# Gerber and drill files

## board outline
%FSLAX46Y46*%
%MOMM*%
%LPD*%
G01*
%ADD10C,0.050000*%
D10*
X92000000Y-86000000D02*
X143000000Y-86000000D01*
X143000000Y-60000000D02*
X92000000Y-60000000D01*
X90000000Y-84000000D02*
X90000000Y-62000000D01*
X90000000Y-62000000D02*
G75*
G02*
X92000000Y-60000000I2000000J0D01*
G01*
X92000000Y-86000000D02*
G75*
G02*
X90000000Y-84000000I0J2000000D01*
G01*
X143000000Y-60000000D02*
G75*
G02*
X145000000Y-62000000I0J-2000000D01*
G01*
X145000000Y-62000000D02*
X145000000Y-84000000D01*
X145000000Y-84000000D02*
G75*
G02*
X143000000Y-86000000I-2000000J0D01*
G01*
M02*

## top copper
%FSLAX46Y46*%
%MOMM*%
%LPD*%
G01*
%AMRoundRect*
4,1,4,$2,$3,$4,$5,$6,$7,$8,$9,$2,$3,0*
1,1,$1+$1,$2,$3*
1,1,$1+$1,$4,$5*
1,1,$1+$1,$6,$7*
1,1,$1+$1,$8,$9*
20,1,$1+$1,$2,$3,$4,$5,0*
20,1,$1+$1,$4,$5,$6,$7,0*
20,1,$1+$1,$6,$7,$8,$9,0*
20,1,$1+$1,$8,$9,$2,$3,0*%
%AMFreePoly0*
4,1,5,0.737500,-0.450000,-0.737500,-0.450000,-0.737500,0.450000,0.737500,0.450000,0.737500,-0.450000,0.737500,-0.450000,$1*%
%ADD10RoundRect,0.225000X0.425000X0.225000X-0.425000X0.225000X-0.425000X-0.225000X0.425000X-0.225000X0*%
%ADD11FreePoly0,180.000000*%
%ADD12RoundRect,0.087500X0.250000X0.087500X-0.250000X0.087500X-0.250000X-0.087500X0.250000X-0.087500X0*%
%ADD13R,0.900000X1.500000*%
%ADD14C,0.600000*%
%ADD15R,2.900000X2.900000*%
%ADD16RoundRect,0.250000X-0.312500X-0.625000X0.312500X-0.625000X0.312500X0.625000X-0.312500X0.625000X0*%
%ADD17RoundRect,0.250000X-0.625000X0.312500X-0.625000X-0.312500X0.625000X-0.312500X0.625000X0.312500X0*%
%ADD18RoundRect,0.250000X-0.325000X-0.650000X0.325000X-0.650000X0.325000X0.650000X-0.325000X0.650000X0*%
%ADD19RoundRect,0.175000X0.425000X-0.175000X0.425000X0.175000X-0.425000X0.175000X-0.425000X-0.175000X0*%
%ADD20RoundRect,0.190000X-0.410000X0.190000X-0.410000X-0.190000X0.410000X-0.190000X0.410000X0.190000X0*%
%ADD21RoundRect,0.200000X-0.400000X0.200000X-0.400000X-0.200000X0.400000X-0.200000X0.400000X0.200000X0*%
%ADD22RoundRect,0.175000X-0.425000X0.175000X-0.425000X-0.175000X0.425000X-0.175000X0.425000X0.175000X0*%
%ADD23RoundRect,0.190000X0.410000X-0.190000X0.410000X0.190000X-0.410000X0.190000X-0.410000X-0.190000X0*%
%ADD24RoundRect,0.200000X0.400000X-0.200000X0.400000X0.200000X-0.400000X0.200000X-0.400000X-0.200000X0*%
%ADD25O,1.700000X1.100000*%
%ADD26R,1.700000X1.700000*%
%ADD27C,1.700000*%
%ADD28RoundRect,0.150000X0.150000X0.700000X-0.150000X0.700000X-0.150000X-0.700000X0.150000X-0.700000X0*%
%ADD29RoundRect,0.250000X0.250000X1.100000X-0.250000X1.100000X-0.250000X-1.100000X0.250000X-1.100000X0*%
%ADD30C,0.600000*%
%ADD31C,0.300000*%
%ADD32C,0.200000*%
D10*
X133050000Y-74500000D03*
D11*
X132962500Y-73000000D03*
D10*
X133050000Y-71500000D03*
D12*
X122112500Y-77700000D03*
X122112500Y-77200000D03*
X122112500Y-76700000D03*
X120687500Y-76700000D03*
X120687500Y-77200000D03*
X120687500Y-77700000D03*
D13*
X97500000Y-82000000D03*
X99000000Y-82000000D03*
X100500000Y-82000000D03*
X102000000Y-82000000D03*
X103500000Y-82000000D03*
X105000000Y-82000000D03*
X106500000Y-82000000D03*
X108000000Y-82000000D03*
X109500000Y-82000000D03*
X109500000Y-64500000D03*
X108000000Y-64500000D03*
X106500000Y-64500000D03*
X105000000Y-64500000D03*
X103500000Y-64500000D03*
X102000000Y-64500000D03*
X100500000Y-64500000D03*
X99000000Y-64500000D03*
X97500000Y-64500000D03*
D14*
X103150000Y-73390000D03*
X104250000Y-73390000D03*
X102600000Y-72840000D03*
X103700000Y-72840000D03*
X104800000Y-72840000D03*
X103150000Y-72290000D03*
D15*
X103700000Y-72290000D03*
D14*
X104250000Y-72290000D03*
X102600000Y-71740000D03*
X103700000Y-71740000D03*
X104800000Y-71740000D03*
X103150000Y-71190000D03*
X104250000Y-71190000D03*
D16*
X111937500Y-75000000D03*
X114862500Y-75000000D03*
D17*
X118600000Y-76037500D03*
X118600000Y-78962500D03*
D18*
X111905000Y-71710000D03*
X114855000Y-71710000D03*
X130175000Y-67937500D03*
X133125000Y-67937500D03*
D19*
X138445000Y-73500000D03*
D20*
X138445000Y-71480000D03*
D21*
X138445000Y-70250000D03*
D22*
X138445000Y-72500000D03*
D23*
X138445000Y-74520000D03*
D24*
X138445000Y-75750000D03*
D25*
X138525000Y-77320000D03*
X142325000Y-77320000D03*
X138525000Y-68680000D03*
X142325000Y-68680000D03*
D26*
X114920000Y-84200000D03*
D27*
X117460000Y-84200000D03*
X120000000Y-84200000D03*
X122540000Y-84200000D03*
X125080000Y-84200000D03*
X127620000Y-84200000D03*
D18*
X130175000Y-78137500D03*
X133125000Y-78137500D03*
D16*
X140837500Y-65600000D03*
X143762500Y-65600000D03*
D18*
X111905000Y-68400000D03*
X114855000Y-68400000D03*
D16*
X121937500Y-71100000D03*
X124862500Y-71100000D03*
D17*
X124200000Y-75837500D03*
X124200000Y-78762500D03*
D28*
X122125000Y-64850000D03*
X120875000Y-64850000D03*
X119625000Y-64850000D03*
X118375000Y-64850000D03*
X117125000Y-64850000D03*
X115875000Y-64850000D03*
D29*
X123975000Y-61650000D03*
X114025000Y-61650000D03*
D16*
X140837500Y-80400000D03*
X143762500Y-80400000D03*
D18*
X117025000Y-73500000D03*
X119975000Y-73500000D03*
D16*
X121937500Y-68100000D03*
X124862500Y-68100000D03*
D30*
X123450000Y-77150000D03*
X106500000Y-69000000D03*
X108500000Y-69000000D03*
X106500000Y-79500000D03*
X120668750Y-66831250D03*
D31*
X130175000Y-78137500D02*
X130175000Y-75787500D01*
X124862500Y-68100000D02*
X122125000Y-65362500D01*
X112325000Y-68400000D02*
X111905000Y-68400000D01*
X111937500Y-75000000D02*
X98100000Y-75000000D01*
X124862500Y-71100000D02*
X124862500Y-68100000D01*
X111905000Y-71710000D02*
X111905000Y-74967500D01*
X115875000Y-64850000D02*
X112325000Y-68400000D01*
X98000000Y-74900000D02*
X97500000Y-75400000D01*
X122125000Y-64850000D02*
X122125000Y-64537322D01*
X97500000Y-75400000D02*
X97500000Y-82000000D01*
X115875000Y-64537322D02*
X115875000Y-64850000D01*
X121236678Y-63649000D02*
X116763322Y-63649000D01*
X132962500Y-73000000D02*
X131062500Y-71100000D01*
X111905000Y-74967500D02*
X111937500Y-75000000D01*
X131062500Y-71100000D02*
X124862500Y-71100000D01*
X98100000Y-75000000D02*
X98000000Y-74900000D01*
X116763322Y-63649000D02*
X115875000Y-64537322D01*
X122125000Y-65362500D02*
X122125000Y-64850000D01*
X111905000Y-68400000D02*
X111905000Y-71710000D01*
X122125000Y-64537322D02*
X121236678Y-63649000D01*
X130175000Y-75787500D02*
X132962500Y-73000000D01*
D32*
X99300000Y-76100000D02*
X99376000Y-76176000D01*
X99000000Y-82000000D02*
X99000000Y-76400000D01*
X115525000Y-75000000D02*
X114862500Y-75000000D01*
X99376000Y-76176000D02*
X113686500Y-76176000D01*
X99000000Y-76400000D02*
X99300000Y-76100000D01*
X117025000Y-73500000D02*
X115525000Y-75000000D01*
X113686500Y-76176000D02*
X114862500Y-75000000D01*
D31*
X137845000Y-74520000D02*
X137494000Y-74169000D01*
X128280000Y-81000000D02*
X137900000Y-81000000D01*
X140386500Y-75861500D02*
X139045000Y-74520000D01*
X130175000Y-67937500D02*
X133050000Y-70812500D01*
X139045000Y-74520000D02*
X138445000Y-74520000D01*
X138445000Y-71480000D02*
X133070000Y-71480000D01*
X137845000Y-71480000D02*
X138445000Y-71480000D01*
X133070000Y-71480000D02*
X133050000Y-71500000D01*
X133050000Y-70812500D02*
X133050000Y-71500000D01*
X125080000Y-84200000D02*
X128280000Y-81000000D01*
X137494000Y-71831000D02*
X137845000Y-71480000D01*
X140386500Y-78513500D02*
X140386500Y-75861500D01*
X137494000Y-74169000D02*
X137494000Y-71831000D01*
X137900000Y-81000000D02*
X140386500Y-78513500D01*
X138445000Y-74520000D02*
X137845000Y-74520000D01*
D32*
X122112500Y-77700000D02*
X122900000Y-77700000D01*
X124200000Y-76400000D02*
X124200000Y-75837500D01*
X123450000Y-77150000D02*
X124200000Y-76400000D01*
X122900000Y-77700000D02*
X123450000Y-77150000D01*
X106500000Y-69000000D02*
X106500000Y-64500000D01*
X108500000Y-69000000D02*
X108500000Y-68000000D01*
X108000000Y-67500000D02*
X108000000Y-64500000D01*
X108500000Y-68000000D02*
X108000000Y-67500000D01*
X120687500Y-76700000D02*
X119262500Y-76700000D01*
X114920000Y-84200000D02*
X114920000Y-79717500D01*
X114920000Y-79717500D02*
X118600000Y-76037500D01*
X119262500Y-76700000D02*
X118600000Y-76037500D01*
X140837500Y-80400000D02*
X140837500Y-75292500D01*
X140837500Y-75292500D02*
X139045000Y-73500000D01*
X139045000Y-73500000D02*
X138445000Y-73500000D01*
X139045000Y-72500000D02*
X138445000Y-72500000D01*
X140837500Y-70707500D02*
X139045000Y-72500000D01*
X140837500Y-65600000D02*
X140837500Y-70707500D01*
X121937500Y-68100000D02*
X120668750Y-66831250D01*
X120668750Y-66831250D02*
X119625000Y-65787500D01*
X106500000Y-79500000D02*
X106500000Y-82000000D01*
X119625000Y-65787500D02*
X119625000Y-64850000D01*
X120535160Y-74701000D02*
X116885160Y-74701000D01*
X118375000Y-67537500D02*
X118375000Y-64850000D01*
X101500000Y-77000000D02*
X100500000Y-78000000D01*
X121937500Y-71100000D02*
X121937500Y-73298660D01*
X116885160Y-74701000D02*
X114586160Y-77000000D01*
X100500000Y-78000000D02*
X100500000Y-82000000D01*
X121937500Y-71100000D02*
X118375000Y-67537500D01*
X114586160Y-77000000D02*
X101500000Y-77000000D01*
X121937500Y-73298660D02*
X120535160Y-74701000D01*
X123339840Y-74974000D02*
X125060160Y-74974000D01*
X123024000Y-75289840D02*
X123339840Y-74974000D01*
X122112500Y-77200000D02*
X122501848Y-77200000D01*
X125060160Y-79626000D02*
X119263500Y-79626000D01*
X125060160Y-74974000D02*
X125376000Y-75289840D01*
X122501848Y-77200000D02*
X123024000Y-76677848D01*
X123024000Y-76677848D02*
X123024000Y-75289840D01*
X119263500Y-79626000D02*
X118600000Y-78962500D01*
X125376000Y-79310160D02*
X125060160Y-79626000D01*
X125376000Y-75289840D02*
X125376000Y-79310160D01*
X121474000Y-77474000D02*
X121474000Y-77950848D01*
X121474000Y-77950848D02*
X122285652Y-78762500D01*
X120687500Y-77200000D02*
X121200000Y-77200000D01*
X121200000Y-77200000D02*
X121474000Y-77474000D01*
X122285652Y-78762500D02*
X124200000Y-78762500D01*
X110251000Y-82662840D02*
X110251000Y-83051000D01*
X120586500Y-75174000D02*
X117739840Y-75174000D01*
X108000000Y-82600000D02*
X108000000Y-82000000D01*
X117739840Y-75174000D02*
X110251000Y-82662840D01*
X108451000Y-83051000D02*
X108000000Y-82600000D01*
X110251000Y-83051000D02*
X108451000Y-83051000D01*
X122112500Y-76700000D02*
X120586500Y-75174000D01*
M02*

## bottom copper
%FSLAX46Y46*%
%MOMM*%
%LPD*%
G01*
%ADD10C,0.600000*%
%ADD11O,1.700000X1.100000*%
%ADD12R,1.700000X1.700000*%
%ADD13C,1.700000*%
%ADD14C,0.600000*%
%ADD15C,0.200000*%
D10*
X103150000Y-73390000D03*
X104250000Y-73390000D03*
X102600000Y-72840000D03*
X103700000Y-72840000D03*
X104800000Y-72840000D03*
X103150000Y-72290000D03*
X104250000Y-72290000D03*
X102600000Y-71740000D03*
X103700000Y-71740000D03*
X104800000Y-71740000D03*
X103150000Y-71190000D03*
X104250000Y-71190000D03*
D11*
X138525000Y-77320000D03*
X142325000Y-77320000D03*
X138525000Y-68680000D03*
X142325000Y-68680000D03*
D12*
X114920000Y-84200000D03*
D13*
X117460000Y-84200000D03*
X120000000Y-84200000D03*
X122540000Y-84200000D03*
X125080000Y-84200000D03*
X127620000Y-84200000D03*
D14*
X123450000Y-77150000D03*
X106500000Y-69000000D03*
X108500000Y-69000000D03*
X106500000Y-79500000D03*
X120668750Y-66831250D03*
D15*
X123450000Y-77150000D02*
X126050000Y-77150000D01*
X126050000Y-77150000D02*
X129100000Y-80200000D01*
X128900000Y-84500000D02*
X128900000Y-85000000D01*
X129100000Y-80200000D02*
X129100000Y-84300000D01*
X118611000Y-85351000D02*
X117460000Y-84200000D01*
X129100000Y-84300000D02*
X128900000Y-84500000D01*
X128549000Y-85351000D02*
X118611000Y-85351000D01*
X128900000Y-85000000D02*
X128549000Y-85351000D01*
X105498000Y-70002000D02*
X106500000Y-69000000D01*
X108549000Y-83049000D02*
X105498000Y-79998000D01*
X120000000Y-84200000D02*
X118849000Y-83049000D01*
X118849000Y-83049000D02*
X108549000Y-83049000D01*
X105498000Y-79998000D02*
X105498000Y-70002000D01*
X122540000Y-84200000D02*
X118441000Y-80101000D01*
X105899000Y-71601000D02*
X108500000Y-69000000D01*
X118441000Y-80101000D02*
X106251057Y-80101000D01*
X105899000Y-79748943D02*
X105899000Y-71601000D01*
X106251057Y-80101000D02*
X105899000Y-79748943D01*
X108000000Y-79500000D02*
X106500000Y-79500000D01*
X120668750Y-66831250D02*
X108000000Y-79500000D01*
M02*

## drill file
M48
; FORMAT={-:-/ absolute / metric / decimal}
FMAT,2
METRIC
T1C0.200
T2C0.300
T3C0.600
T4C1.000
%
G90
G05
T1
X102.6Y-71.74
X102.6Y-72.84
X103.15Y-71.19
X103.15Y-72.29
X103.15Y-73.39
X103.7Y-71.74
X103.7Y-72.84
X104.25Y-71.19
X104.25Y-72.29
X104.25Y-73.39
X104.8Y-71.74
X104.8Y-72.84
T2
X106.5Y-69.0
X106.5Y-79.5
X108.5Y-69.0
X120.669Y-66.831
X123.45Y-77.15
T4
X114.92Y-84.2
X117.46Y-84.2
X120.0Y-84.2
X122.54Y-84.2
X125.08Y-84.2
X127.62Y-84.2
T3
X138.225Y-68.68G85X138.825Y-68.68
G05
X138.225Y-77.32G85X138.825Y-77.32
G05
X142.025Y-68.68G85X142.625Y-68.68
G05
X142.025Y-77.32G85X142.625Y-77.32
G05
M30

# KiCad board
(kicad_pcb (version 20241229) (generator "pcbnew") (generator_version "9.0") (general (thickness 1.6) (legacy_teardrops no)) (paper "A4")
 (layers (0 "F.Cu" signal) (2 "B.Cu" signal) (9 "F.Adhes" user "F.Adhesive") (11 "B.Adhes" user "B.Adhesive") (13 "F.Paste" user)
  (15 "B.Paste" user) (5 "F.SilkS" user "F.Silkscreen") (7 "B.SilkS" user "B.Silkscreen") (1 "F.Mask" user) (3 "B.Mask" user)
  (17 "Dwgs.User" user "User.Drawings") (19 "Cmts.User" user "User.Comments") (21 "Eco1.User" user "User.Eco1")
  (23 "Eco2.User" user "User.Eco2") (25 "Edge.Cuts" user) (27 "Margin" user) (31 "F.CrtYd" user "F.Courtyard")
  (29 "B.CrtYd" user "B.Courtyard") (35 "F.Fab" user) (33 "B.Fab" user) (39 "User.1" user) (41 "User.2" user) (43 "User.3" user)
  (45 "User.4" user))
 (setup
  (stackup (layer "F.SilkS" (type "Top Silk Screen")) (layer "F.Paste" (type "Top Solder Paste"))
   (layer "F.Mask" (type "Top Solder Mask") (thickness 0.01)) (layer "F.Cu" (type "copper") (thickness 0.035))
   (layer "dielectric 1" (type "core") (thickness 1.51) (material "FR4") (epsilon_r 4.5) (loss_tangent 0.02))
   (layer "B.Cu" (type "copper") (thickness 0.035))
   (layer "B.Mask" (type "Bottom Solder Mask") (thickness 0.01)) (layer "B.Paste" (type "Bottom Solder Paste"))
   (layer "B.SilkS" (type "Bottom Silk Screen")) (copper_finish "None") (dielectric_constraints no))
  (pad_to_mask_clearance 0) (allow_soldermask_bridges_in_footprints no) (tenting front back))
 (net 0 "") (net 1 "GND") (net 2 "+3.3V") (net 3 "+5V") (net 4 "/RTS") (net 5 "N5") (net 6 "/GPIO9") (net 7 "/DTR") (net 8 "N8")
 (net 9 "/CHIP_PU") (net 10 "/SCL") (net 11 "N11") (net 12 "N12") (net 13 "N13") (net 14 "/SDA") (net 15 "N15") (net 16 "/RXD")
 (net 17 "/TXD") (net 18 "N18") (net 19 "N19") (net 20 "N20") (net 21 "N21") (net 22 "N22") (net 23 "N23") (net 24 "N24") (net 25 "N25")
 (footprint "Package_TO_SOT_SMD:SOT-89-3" (layer "F.Cu") (at 131.1 73 180)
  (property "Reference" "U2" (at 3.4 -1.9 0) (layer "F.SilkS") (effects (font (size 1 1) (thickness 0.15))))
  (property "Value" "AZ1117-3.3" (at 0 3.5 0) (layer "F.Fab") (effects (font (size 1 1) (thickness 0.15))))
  (pad "1" smd roundrect (at -1.95 -1.5 180) (size 1.3 0.9) (layers "F.Cu" "F.Mask" "F.Paste") (roundrect_rratio 0.25) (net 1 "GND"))
  (pad "2" smd custom (at -1.8625 0 180) (size 1.475 0.9) (layers "F.Cu" "F.Mask" "F.Paste") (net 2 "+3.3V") (zone_connect 2)
   (thermal_bridge_angle 45) (options (clearance outline) (anchor rect)) (primitives))
  (pad "3" smd roundrect (at -1.95 1.5 180) (size 1.3 0.9) (layers "F.Cu" "F.Mask" "F.Paste") (roundrect_rratio 0.25) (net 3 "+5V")))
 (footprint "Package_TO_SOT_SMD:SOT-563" (layer "F.Cu") (at 121.4 77.2 180)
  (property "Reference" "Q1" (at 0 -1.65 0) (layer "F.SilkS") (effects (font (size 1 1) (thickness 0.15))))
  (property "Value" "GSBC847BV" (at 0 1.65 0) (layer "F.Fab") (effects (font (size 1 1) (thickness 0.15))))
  (pad "1" smd roundrect (at -0.7125 -0.5 180) (size 0.675 0.35) (layers "F.Cu" "F.Mask" "F.Paste") (roundrect_rratio 0.25) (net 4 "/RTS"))
  (pad "2" smd roundrect (at -0.7125 0 180) (size 0.675 0.35) (layers "F.Cu" "F.Mask" "F.Paste") (roundrect_rratio 0.25) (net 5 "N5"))
  (pad "3" smd roundrect (at -0.7125 0.5 180) (size 0.675 0.35) (layers "F.Cu" "F.Mask" "F.Paste") (roundrect_rratio 0.25) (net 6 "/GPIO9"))
  (pad "4" smd roundrect (at 0.7125 0.5 180) (size 0.675 0.35) (layers "F.Cu" "F.Mask" "F.Paste") (roundrect_rratio 0.25) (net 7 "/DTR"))
  (pad "5" smd roundrect (at 0.7125 0 180) (size 0.675 0.35) (layers "F.Cu" "F.Mask" "F.Paste") (roundrect_rratio 0.25) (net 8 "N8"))
  (pad "6" smd roundrect (at 0.7125 -0.5 180) (size 0.675 0.35) (layers "F.Cu" "F.Mask" "F.Paste") (roundrect_rratio 0.25)
   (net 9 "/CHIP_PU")))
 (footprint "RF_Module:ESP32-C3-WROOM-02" (layer "F.Cu") (at 103.5 73.25 90)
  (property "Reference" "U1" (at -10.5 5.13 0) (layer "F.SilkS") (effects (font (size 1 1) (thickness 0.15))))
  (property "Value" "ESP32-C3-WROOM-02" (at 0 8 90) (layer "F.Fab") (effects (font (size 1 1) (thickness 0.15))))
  (pad "" smd rect (at -0.14 -0.9 90) (size 0.7 0.7) (layers "F.Paste"))
  (pad "" smd rect (at -0.14 0.2 90) (size 0.7 0.7) (layers "F.Paste"))
  (pad "" smd rect (at -0.14 1.3 90) (size 0.7 0.7) (layers "F.Paste"))
  (pad "" smd rect (at 0.96 -0.9 90) (size 0.7 0.7) (layers "F.Paste"))
  (pad "" smd rect (at 0.96 0.2 90) (size 0.7 0.7) (layers "F.Paste"))
  (pad "" smd rect (at 0.96 1.3 90) (size 0.7 0.7) (layers "F.Paste"))
  (pad "" smd rect (at 2.06 -0.9 90) (size 0.7 0.7) (layers "F.Paste"))
  (pad "" smd rect (at 2.06 0.2 90) (size 0.7 0.7) (layers "F.Paste"))
  (pad "" smd rect (at 2.06 1.3 90) (size 0.7 0.7) (layers "F.Paste"))
  (pad "1" smd rect (at -8.75 -6 90) (size 1.5 0.9) (layers "F.Cu" "F.Mask" "F.Paste") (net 2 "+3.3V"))
  (pad "2" smd rect (at -8.75 -4.5 90) (size 1.5 0.9) (layers "F.Cu" "F.Mask" "F.Paste") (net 9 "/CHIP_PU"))
  (pad "3" smd rect (at -8.75 -3 90) (size 1.5 0.9) (layers "F.Cu" "F.Mask" "F.Paste") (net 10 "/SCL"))
  (pad "4" smd rect (at -8.75 -1.5 90) (size 1.5 0.9) (layers "F.Cu" "F.Mask" "F.Paste") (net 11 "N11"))
  (pad "5" smd rect (at -8.75 0 90) (size 1.5 0.9) (layers "F.Cu" "F.Mask" "F.Paste") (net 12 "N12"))
  (pad "6" smd rect (at -8.75 1.5 90) (size 1.5 0.9) (layers "F.Cu" "F.Mask" "F.Paste") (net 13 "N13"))
  (pad "7" smd rect (at -8.75 3 90) (size 1.5 0.9) (layers "F.Cu" "F.Mask" "F.Paste") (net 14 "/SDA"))
  (pad "8" smd rect (at -8.75 4.5 90) (size 1.5 0.9) (layers "F.Cu" "F.Mask" "F.Paste") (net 6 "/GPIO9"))
  (pad "9" smd rect (at -8.75 6 90) (size 1.5 0.9) (layers "F.Cu" "F.Mask" "F.Paste") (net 1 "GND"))
  (pad "10" smd rect (at 8.75 6 90) (size 1.5 0.9) (layers "F.Cu" "F.Mask" "F.Paste") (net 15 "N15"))
  (pad "11" smd rect (at 8.75 4.5 90) (size 1.5 0.9) (layers "F.Cu" "F.Mask" "F.Paste") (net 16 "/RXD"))
  (pad "12" smd rect (at 8.75 3 90) (size 1.5 0.9) (layers "F.Cu" "F.Mask" "F.Paste") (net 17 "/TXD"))
  (pad "13" smd rect (at 8.75 1.5 90) (size 1.5 0.9) (layers "F.Cu" "F.Mask" "F.Paste") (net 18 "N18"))
  (pad "14" smd rect (at 8.75 0 90) (size 1.5 0.9) (layers "F.Cu" "F.Mask" "F.Paste") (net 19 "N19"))
  (pad "15" smd rect (at 8.75 -1.5 90) (size 1.5 0.9) (layers "F.Cu" "F.Mask" "F.Paste") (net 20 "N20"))
  (pad "16" smd rect (at 8.75 -3 90) (size 1.5 0.9) (layers "F.Cu" "F.Mask" "F.Paste") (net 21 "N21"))
  (pad "17" smd rect (at 8.75 -4.5 90) (size 1.5 0.9) (layers "F.Cu" "F.Mask" "F.Paste") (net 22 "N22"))
  (pad "18" smd rect (at 8.75 -6 90) (size 1.5 0.9) (layers "F.Cu" "F.Mask" "F.Paste") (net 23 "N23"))
  (pad "19" thru_hole circle (at -0.14 -0.35 90) (size 0.6 0.6) (drill 0.2) (layers "*.Cu" "F.Mask") (remove_unused_layers no) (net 1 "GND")
   (zone_connect 2))
  (pad "19" thru_hole circle (at -0.14 0.75 90) (size 0.6 0.6) (drill 0.2) (layers "*.Cu" "F.Mask") (remove_unused_layers no) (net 1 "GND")
   (zone_connect 2))
  (pad "19" thru_hole circle (at 0.41 -0.9 90) (size 0.6 0.6) (drill 0.2) (layers "*.Cu" "F.Mask") (remove_unused_layers no) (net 1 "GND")
   (zone_connect 2))
  (pad "19" thru_hole circle (at 0.41 0.2 90) (size 0.6 0.6) (drill 0.2) (layers "*.Cu" "F.Mask") (remove_unused_layers no) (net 1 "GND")
   (zone_connect 2))
  (pad "19" thru_hole circle (at 0.41 1.3 90) (size 0.6 0.6) (drill 0.2) (layers "*.Cu" "F.Mask") (remove_unused_layers no) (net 1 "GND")
   (zone_connect 2))
  (pad "19" thru_hole circle (at 0.96 -0.35 90) (size 0.6 0.6) (drill 0.2) (layers "*.Cu" "F.Mask") (remove_unused_layers no) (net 1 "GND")
   (zone_connect 2))
  (pad "19" smd rect (at 0.96 0.2 90) (size 2.9 2.9) (layers "F.Cu" "F.Mask") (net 1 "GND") (zone_connect 2))
  (pad "19" thru_hole circle (at 0.96 0.75 90) (size 0.6 0.6) (drill 0.2) (layers "*.Cu" "F.Mask") (remove_unused_layers no) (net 1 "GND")
   (zone_connect 2))
  (pad "19" thru_hole circle (at 1.51 -0.9 90) (size 0.6 0.6) (drill 0.2) (layers "*.Cu" "F.Mask") (remove_unused_layers no) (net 1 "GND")
   (zone_connect 2))
  (pad "19" thru_hole circle (at 1.51 0.2 90) (size 0.6 0.6) (drill 0.2) (layers "*.Cu" "F.Mask") (remove_unused_layers no) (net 1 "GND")
   (zone_connect 2))
  (pad "19" thru_hole circle (at 1.51 1.3 90) (size 0.6 0.6) (drill 0.2) (layers "*.Cu" "F.Mask") (remove_unused_layers no) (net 1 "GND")
   (zone_connect 2))
  (pad "19" thru_hole circle (at 2.06 -0.35 90) (size 0.6 0.6) (drill 0.2) (layers "*.Cu" "F.Mask") (remove_unused_layers no) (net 1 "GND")
   (zone_connect 2))
  (pad "19" thru_hole circle (at 2.06 0.75 90) (size 0.6 0.6) (drill 0.2) (layers "*.Cu" "F.Mask") (remove_unused_layers no) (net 1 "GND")
   (zone_connect 2))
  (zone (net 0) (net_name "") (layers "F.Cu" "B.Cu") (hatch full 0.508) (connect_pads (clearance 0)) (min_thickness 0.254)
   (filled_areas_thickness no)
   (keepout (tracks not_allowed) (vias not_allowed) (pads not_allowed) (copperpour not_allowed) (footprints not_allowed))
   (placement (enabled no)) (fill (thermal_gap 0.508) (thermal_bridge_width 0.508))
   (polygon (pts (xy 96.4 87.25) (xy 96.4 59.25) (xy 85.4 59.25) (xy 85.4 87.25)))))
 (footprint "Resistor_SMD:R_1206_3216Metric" (layer "F.Cu") (at 113.4 75)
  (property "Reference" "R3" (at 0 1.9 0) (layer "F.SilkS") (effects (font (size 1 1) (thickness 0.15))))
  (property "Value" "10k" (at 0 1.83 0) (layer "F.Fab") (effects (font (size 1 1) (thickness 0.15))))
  (pad "1" smd roundrect (at -1.4625 0) (size 1.125 1.75) (layers "F.Cu" "F.Mask" "F.Paste") (roundrect_rratio 0.222222) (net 2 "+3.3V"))
  (pad "2" smd roundrect (at 1.4625 0) (size 1.125 1.75) (layers "F.Cu" "F.Mask" "F.Paste") (roundrect_rratio 0.222222) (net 9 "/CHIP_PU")))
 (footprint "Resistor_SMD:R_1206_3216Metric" (layer "F.Cu") (at 118.6 77.5 -90)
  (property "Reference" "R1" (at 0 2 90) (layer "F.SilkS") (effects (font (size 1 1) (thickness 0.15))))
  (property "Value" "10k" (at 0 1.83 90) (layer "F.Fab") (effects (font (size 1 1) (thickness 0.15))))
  (pad "1" smd roundrect (at -1.4625 0 270) (size 1.125 1.75) (layers "F.Cu" "F.Mask" "F.Paste") (roundrect_rratio 0.222222) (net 7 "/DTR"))
  (pad "2" smd roundrect (at 1.4625 0 270) (size 1.125 1.75) (layers "F.Cu" "F.Mask" "F.Paste") (roundrect_rratio 0.222222) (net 5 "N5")))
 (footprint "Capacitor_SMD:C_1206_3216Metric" (layer "F.Cu") (at 113.38 71.71)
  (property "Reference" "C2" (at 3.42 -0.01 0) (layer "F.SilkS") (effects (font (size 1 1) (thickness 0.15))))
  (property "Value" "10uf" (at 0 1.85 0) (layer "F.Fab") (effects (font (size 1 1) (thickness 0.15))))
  (pad "1" smd roundrect (at -1.475 0) (size 1.15 1.8) (layers "F.Cu" "F.Mask" "F.Paste") (roundrect_rratio 0.217391) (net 2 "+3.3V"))
  (pad "2" smd roundrect (at 1.475 0) (size 1.15 1.8) (layers "F.Cu" "F.Mask" "F.Paste") (roundrect_rratio 0.217391) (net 1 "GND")))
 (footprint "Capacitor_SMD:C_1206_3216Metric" (layer "F.Cu") (at 131.65 67.9375)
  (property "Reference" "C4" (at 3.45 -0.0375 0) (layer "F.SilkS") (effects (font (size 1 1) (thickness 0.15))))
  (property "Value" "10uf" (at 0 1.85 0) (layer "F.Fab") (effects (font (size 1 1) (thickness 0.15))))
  (pad "1" smd roundrect (at -1.475 0) (size 1.15 1.8) (layers "F.Cu" "F.Mask" "F.Paste") (roundrect_rratio 0.217391) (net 3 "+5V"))
  (pad "2" smd roundrect (at 1.475 0) (size 1.15 1.8) (layers "F.Cu" "F.Mask" "F.Paste") (roundrect_rratio 0.217391) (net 1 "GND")))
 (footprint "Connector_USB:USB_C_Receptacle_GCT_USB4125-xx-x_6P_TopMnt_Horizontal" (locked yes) (layer "F.Cu") (at 141.525 73 90)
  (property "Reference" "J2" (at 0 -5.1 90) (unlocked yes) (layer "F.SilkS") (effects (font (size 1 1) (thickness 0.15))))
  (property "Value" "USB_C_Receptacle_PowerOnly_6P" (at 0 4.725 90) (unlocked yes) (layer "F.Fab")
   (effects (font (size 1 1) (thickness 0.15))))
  (pad "A5" smd roundrect (at -0.5 -3.08 90) (size 0.7 1.2) (layers "F.Cu" "F.Mask" "F.Paste") (roundrect_rratio 0.25) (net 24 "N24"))
  (pad "A9" smd roundrect (at 1.52 -3.08 270) (size 0.76 1.2) (layers "F.Cu" "F.Mask" "F.Paste") (roundrect_rratio 0.25) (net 3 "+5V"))
  (pad "A12" smd roundrect (at 2.75 -3.08 270) (size 0.8 1.2) (layers "F.Cu" "F.Mask" "F.Paste") (roundrect_rratio 0.25) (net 1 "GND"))
  (pad "B5" smd roundrect (at 0.5 -3.08 270) (size 0.7 1.2) (layers "F.Cu" "F.Mask" "F.Paste") (roundrect_rratio 0.25) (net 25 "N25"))
  (pad "B9" smd roundrect (at -1.52 -3.08 90) (size 0.76 1.2) (layers "F.Cu" "F.Mask" "F.Paste") (roundrect_rratio 0.25) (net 3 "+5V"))
  (pad "B12" smd roundrect (at -2.75 -3.08 90) (size 0.8 1.2) (layers "F.Cu" "F.Mask" "F.Paste") (roundrect_rratio 0.25) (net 1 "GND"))
  (pad "S1" thru_hole oval (at -4.32 -3 90) (size 1.1 1.7) (drill oval 0.6 1.2) (layers "*.Cu" "*.Mask" "F.Paste") (remove_unused_layers no)
   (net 1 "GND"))
  (pad "S1" thru_hole oval (at -4.32 0.8 90) (size 1.1 1.7) (drill oval 0.6 1.2) (layers "*.Cu" "*.Mask" "F.Paste")
   (remove_unused_layers no) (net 1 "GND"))
  (pad "S1" thru_hole oval (at 4.32 -3 90) (size 1.1 1.7) (drill oval 0.6 1.2) (layers "*.Cu" "*.Mask" "F.Paste") (remove_unused_layers no)
   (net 1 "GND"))
  (pad "S1" thru_hole oval (at 4.32 0.8 90) (size 1.1 1.7) (drill oval 0.6 1.2) (layers "*.Cu" "*.Mask" "F.Paste") (remove_unused_layers no)
   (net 1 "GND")))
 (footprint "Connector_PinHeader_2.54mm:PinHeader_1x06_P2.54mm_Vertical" (layer "F.Cu") (at 114.92 84.2 90)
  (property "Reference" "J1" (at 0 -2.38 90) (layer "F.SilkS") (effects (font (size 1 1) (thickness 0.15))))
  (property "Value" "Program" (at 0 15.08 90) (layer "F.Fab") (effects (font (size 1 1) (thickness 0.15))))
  (pad "1" thru_hole rect (at 0 0 90) (size 1.7 1.7) (drill 1) (layers "*.Cu" "*.Mask") (remove_unused_layers no) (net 7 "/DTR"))
  (pad "2" thru_hole circle (at 0 2.54 90) (size 1.7 1.7) (drill 1) (layers "*.Cu" "*.Mask") (remove_unused_layers no) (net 4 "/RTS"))
  (pad "3" thru_hole circle (at 0 5.08 90) (size 1.7 1.7) (drill 1) (layers "*.Cu" "*.Mask") (remove_unused_layers no) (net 17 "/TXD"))
  (pad "4" thru_hole circle (at 0 7.62 90) (size 1.7 1.7) (drill 1) (layers "*.Cu" "*.Mask") (remove_unused_layers no) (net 16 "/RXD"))
  (pad "5" thru_hole circle (at 0 10.16 90) (size 1.7 1.7) (drill 1) (layers "*.Cu" "*.Mask") (remove_unused_layers no) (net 3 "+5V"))
  (pad "6" thru_hole circle (at 0 12.7 90) (size 1.7 1.7) (drill 1) (layers "*.Cu" "*.Mask") (remove_unused_layers no) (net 1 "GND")))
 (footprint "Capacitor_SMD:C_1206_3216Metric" (layer "F.Cu") (at 131.65 78.1375)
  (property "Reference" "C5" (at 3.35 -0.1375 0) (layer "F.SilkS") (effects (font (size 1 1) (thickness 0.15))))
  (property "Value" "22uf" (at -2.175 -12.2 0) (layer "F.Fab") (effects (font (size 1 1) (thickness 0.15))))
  (pad "1" smd roundrect (at -1.475 0) (size 1.15 1.8) (layers "F.Cu" "F.Mask" "F.Paste") (roundrect_rratio 0.217391) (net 2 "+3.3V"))
  (pad "2" smd roundrect (at 1.475 0) (size 1.15 1.8) (layers "F.Cu" "F.Mask" "F.Paste") (roundrect_rratio 0.217391) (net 1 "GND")))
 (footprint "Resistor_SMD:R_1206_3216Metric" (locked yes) (layer "F.Cu") (at 142.3 65.6)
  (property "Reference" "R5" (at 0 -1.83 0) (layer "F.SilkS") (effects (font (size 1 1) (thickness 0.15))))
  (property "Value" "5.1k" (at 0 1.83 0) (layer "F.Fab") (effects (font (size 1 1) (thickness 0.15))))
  (pad "1" smd roundrect (at -1.4625 0) (size 1.125 1.75) (layers "F.Cu" "F.Mask" "F.Paste") (roundrect_rratio 0.222222) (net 25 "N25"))
  (pad "2" smd roundrect (at 1.4625 0) (size 1.125 1.75) (layers "F.Cu" "F.Mask" "F.Paste") (roundrect_rratio 0.222222) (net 1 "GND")))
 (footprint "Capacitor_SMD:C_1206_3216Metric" (layer "F.Cu") (at 113.38 68.4)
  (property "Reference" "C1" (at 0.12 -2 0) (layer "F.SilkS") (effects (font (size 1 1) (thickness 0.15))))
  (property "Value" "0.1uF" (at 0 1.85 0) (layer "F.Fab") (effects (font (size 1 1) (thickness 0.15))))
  (pad "1" smd roundrect (at -1.475 0) (size 1.15 1.8) (layers "F.Cu" "F.Mask" "F.Paste") (roundrect_rratio 0.217391) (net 2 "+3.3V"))
  (pad "2" smd roundrect (at 1.475 0) (size 1.15 1.8) (layers "F.Cu" "F.Mask" "F.Paste") (roundrect_rratio 0.217391) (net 1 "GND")))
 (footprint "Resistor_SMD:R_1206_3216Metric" (layer "F.Cu") (at 123.4 71.1)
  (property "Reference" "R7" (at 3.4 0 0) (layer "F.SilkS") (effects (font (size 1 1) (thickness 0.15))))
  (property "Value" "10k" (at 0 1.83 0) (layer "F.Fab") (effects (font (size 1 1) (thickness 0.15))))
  (pad "1" smd roundrect (at -1.4625 0) (size 1.125 1.75) (layers "F.Cu" "F.Mask" "F.Paste") (roundrect_rratio 0.222222) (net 10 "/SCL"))
  (pad "2" smd roundrect (at 1.4625 0) (size 1.125 1.75) (layers "F.Cu" "F.Mask" "F.Paste") (roundrect_rratio 0.222222) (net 2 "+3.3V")))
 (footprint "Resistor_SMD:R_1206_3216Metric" (layer "F.Cu") (at 124.2 77.3 -90)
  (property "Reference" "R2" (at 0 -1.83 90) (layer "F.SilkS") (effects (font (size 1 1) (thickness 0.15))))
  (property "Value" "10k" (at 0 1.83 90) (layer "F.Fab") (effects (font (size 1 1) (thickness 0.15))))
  (pad "1" smd roundrect (at -1.4625 0 270) (size 1.125 1.75) (layers "F.Cu" "F.Mask" "F.Paste") (roundrect_rratio 0.222222) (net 4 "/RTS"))
  (pad "2" smd roundrect (at 1.4625 0 270) (size 1.125 1.75) (layers "F.Cu" "F.Mask" "F.Paste") (roundrect_rratio 0.222222) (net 8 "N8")))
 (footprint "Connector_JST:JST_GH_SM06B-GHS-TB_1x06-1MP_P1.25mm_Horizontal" (layer "F.Cu") (at 119 63 180)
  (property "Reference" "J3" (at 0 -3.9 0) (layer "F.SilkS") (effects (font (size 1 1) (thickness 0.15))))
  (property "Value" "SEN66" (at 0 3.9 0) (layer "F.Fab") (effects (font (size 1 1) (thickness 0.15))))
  (pad "1" smd roundrect (at -3.125 -1.85 180) (size 0.6 1.7) (layers "F.Cu" "F.Mask" "F.Paste") (roundrect_rratio 0.25) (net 2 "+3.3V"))
  (pad "2" smd roundrect (at -1.875 -1.85 180) (size 0.6 1.7) (layers "F.Cu" "F.Mask" "F.Paste") (roundrect_rratio 0.25) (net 1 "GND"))
  (pad "3" smd roundrect (at -0.625 -1.85 180) (size 0.6 1.7) (layers "F.Cu" "F.Mask" "F.Paste") (roundrect_rratio 0.25) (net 14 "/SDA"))
  (pad "4" smd roundrect (at 0.625 -1.85 180) (size 0.6 1.7) (layers "F.Cu" "F.Mask" "F.Paste") (roundrect_rratio 0.25) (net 10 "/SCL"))
  (pad "5" smd roundrect (at 1.875 -1.85 180) (size 0.6 1.7) (layers "F.Cu" "F.Mask" "F.Paste") (roundrect_rratio 0.25) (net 1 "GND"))
  (pad "6" smd roundrect (at 3.125 -1.85 180) (size 0.6 1.7) (layers "F.Cu" "F.Mask" "F.Paste") (roundrect_rratio 0.25) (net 2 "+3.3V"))
  (pad "MP" smd roundrect (at -4.975 1.35 180) (size 1 2.7) (layers "F.Cu" "F.Mask" "F.Paste") (roundrect_rratio 0.25))
  (pad "MP" smd roundrect (at 4.975 1.35 180) (size 1 2.7) (layers "F.Cu" "F.Mask" "F.Paste") (roundrect_rratio 0.25)))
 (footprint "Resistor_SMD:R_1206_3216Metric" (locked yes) (layer "F.Cu") (at 142.3 80.4)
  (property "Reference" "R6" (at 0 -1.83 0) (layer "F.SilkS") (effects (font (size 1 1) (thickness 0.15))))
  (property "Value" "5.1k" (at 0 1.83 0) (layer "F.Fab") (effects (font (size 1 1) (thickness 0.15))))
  (pad "1" smd roundrect (at -1.4625 0) (size 1.125 1.75) (layers "F.Cu" "F.Mask" "F.Paste") (roundrect_rratio 0.222222) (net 24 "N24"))
  (pad "2" smd roundrect (at 1.4625 0) (size 1.125 1.75) (layers "F.Cu" "F.Mask" "F.Paste") (roundrect_rratio 0.222222) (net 1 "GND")))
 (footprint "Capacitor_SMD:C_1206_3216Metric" (layer "F.Cu") (at 118.5 73.5)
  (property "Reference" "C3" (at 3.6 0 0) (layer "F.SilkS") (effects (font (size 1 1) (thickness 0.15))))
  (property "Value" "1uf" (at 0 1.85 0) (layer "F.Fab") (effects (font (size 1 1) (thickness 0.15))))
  (pad "1" smd roundrect (at -1.475 0) (size 1.15 1.8) (layers "F.Cu" "F.Mask" "F.Paste") (roundrect_rratio 0.217391) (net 9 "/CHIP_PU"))
  (pad "2" smd roundrect (at 1.475 0) (size 1.15 1.8) (layers "F.Cu" "F.Mask" "F.Paste") (roundrect_rratio 0.217391) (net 1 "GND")))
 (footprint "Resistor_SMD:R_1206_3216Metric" (layer "F.Cu") (at 123.4 68.1)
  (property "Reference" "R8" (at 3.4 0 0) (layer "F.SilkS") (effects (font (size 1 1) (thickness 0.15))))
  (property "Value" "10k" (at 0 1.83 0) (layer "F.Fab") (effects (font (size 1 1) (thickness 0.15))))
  (pad "1" smd roundrect (at -1.4625 0) (size 1.125 1.75) (layers "F.Cu" "F.Mask" "F.Paste") (roundrect_rratio 0.222222) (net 14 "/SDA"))
  (pad "2" smd roundrect (at 1.4625 0) (size 1.125 1.75) (layers "F.Cu" "F.Mask" "F.Paste") (roundrect_rratio 0.222222) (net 2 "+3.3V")))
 (gr_line (start 92 86) (end 143 86) (stroke (width 0.05) (type default)) (layer "Edge.Cuts"))
 (gr_line (start 143 60) (end 92 60) (stroke (width 0.05) (type default)) (layer "Edge.Cuts"))
 (gr_line (start 90 84) (end 90 62) (stroke (width 0.05) (type default)) (layer "Edge.Cuts"))
 (gr_arc (start 90 62) (mid 90.585786 60.585786) (end 92 60) (stroke (width 0.05) (type default)) (layer "Edge.Cuts"))
 (gr_arc (start 92 86) (mid 90.585786 85.414214) (end 90 84) (stroke (width 0.05) (type default)) (layer "Edge.Cuts"))
 (gr_arc (start 143 60) (mid 144.414214 60.585786) (end 145 62) (stroke (width 0.05) (type default)) (layer "Edge.Cuts"))
 (gr_line (start 145 62) (end 145 84) (stroke (width 0.05) (type default)) (layer "Edge.Cuts"))
 (gr_arc (start 145 84) (mid 144.414214 85.414214) (end 143 86) (stroke (width 0.05) (type default)) (layer "Edge.Cuts"))
 (segment (start 130.175 78.1375) (end 130.175 75.7875) (width 0.3) (layer "F.Cu") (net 2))
 (segment (start 124.8625 68.1) (end 122.125 65.3625) (width 0.3) (layer "F.Cu") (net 2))
 (segment (start 112.325 68.4) (end 111.905 68.4) (width 0.3) (layer "F.Cu") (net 2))
 (segment (start 111.9375 75) (end 98.1 75) (width 0.3) (layer "F.Cu") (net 2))
 (segment (start 124.8625 71.1) (end 124.8625 68.1) (width 0.3) (layer "F.Cu") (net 2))
 (segment (start 111.905 71.71) (end 111.905 74.9675) (width 0.3) (layer "F.Cu") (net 2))
 (segment (start 115.875 64.85) (end 112.325 68.4) (width 0.3) (layer "F.Cu") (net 2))
 (segment (start 98 74.9) (end 97.5 75.4) (width 0.3) (layer "F.Cu") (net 2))
 (segment (start 122.125 64.85) (end 122.125 64.537322) (width 0.3) (layer "F.Cu") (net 2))
 (segment (start 97.5 75.4) (end 97.5 82) (width 0.3) (layer "F.Cu") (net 2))
 (segment (start 115.875 64.537322) (end 115.875 64.85) (width 0.3) (layer "F.Cu") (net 2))
 (segment (start 121.236678 63.649) (end 116.763322 63.649) (width 0.3) (layer "F.Cu") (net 2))
 (segment (start 132.9625 73) (end 131.0625 71.1) (width 0.3) (layer "F.Cu") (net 2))
 (segment (start 111.905 74.9675) (end 111.9375 75) (width 0.3) (layer "F.Cu") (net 2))
 (segment (start 131.0625 71.1) (end 124.8625 71.1) (width 0.3) (layer "F.Cu") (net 2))
 (segment (start 98.1 75) (end 98 74.9) (width 0.3) (layer "F.Cu") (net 2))
 (segment (start 116.763322 63.649) (end 115.875 64.537322) (width 0.3) (layer "F.Cu") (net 2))
 (segment (start 122.125 65.3625) (end 122.125 64.85) (width 0.3) (layer "F.Cu") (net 2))
 (segment (start 111.905 68.4) (end 111.905 71.71) (width 0.3) (layer "F.Cu") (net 2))
 (segment (start 122.125 64.537322) (end 121.236678 63.649) (width 0.3) (layer "F.Cu") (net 2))
 (segment (start 130.175 75.7875) (end 132.9625 73) (width 0.3) (layer "F.Cu") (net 2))
 (segment (start 99.3 76.1) (end 99.376 76.176) (width 0.2) (layer "F.Cu") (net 9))
 (segment (start 99 82) (end 99 76.4) (width 0.2) (layer "F.Cu") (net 9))
 (segment (start 115.525 75) (end 114.8625 75) (width 0.2) (layer "F.Cu") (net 9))
 (segment (start 99.376 76.176) (end 113.6865 76.176) (width 0.2) (layer "F.Cu") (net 9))
 (segment (start 99 76.4) (end 99.3 76.1) (width 0.2) (layer "F.Cu") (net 9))
 (segment (start 117.025 73.5) (end 115.525 75) (width 0.2) (layer "F.Cu") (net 9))
 (segment (start 113.6865 76.176) (end 114.8625 75) (width 0.2) (layer "F.Cu") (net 9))
 (segment (start 137.845 74.52) (end 137.494 74.169) (width 0.3) (layer "F.Cu") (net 3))
 (segment (start 128.28 81) (end 137.9 81) (width 0.3) (layer "F.Cu") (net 3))
 (segment (start 140.3865 75.8615) (end 139.045 74.52) (width 0.3) (layer "F.Cu") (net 3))
 (segment (start 130.175 67.9375) (end 133.05 70.8125) (width 0.3) (layer "F.Cu") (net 3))
 (segment (start 139.045 74.52) (end 138.445 74.52) (width 0.3) (layer "F.Cu") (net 3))
 (segment (start 138.445 71.48) (end 133.07 71.48) (width 0.3) (layer "F.Cu") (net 3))
 (segment (start 137.845 71.48) (end 138.445 71.48) (width 0.3) (layer "F.Cu") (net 3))
 (segment (start 133.07 71.48) (end 133.05 71.5) (width 0.3) (layer "F.Cu") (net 3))
 (segment (start 133.05 70.8125) (end 133.05 71.5) (width 0.3) (layer "F.Cu") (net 3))
 (segment (start 125.08 84.2) (end 128.28 81) (width 0.3) (layer "F.Cu") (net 3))
 (segment (start 137.494 71.831) (end 137.845 71.48) (width 0.3) (layer "F.Cu") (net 3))
 (segment (start 140.3865 78.5135) (end 140.3865 75.8615) (width 0.3) (layer "F.Cu") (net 3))
 (segment (start 137.494 74.169) (end 137.494 71.831) (width 0.3) (layer "F.Cu") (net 3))
 (segment (start 137.9 81) (end 140.3865 78.5135) (width 0.3) (layer "F.Cu") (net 3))
 (segment (start 138.445 74.52) (end 137.845 74.52) (width 0.3) (layer "F.Cu") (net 3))
 (segment (start 122.1125 77.7) (end 122.9 77.7) (width 0.2) (layer "F.Cu") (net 4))
 (segment (start 124.2 76.4) (end 124.2 75.8375) (width 0.2) (layer "F.Cu") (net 4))
 (segment (start 123.45 77.15) (end 124.2 76.4) (width 0.2) (layer "F.Cu") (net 4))
 (segment (start 122.9 77.7) (end 123.45 77.15) (width 0.2) (layer "F.Cu") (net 4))
 (via (at 123.45 77.15) (size 0.6) (drill 0.3) (layers "F.Cu" "B.Cu") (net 4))
 (segment (start 123.45 77.15) (end 126.05 77.15) (width 0.2) (layer "B.Cu") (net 4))
 (segment (start 126.05 77.15) (end 129.1 80.2) (width 0.2) (layer "B.Cu") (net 4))
 (segment (start 128.9 84.5) (end 128.9 85) (width 0.2) (layer "B.Cu") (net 4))
 (segment (start 129.1 80.2) (end 129.1 84.3) (width 0.2) (layer "B.Cu") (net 4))
 (segment (start 118.611 85.351) (end 117.46 84.2) (width 0.2) (layer "B.Cu") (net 4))
 (segment (start 129.1 84.3) (end 128.9 84.5) (width 0.2) (layer "B.Cu") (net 4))
 (segment (start 128.549 85.351) (end 118.611 85.351) (width 0.2) (layer "B.Cu") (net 4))
 (segment (start 128.9 85) (end 128.549 85.351) (width 0.2) (layer "B.Cu") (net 4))
 (segment (start 106.5 69) (end 106.5 64.5) (width 0.2) (layer "F.Cu") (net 17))
 (via (at 106.5 69) (size 0.6) (drill 0.3) (layers "F.Cu" "B.Cu") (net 17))
 (segment (start 105.498 70.002) (end 106.5 69) (width 0.2) (layer "B.Cu") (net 17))
 (segment (start 108.549 83.049) (end 105.498 79.998) (width 0.2) (layer "B.Cu") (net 17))
 (segment (start 120 84.2) (end 118.849 83.049) (width 0.2) (layer "B.Cu") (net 17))
 (segment (start 118.849 83.049) (end 108.549 83.049) (width 0.2) (layer "B.Cu") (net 17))
 (segment (start 105.498 79.998) (end 105.498 70.002) (width 0.2) (layer "B.Cu") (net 17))
 (segment (start 108.5 69) (end 108.5 68) (width 0.2) (layer "F.Cu") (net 16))
 (segment (start 108 67.5) (end 108 64.5) (width 0.2) (layer "F.Cu") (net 16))
 (segment (start 108.5 68) (end 108 67.5) (width 0.2) (layer "F.Cu") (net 16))
 (via (at 108.5 69) (size 0.6) (drill 0.3) (layers "F.Cu" "B.Cu") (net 16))
 (segment (start 122.54 84.2) (end 118.441 80.101) (width 0.2) (layer "B.Cu") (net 16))
 (segment (start 105.899 71.601) (end 108.5 69) (width 0.2) (layer "B.Cu") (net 16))
 (segment (start 118.441 80.101) (end 106.251057 80.101) (width 0.2) (layer "B.Cu") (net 16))
 (segment (start 105.899 79.748943) (end 105.899 71.601) (width 0.2) (layer "B.Cu") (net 16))
 (segment (start 106.251057 80.101) (end 105.899 79.748943) (width 0.2) (layer "B.Cu") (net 16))
 (segment (start 120.6875 76.7) (end 119.2625 76.7) (width 0.2) (layer "F.Cu") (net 7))
 (segment (start 114.92 84.2) (end 114.92 79.7175) (width 0.2) (layer "F.Cu") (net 7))
 (segment (start 114.92 79.7175) (end 118.6 76.0375) (width 0.2) (layer "F.Cu") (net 7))
 (segment (start 119.2625 76.7) (end 118.6 76.0375) (width 0.2) (layer "F.Cu") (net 7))
 (segment (start 140.8375 80.4) (end 140.8375 75.2925) (width 0.2) (layer "F.Cu") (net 24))
 (segment (start 140.8375 75.2925) (end 139.045 73.5) (width 0.2) (layer "F.Cu") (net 24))
 (segment (start 139.045 73.5) (end 138.445 73.5) (width 0.2) (layer "F.Cu") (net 24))
 (segment (start 139.045 72.5) (end 138.445 72.5) (width 0.2) (layer "F.Cu") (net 25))
 (segment (start 140.8375 70.7075) (end 139.045 72.5) (width 0.2) (layer "F.Cu") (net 25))
 (segment (start 140.8375 65.6) (end 140.8375 70.7075) (width 0.2) (layer "F.Cu") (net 25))
 (segment (start 121.9375 68.1) (end 120.66875 66.83125) (width 0.2) (layer "F.Cu") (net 14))
 (segment (start 120.66875 66.83125) (end 119.625 65.7875) (width 0.2) (layer "F.Cu") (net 14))
 (segment (start 106.5 79.5) (end 106.5 82) (width 0.2) (layer "F.Cu") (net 14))
 (segment (start 119.625 65.7875) (end 119.625 64.85) (width 0.2) (layer "F.Cu") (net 14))
 (via (at 106.5 79.5) (size 0.6) (drill 0.3) (layers "F.Cu" "B.Cu") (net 14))
 (via (at 120.66875 66.83125) (size 0.6) (drill 0.3) (layers "F.Cu" "B.Cu") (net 14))
 (segment (start 108 79.5) (end 106.5 79.5) (width 0.2) (layer "B.Cu") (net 14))
 (segment (start 120.66875 66.83125) (end 108 79.5) (width 0.2) (layer "B.Cu") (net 14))
 (segment (start 120.53516 74.701) (end 116.88516 74.701) (width 0.2) (layer "F.Cu") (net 10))
 (segment (start 118.375 67.5375) (end 118.375 64.85) (width 0.2) (layer "F.Cu") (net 10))
 (segment (start 101.5 77) (end 100.5 78) (width 0.2) (layer "F.Cu") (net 10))
 (segment (start 121.9375 71.1) (end 121.9375 73.29866) (width 0.2) (layer "F.Cu") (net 10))
 (segment (start 116.88516 74.701) (end 114.58616 77) (width 0.2) (layer "F.Cu") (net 10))
 (segment (start 100.5 78) (end 100.5 82) (width 0.2) (layer "F.Cu") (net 10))
 (segment (start 121.9375 71.1) (end 118.375 67.5375) (width 0.2) (layer "F.Cu") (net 10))
 (segment (start 114.58616 77) (end 101.5 77) (width 0.2) (layer "F.Cu") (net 10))
 (segment (start 121.9375 73.29866) (end 120.53516 74.701) (width 0.2) (layer "F.Cu") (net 10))
 (segment (start 123.33984 74.974) (end 125.06016 74.974) (width 0.2) (layer "F.Cu") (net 5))
 (segment (start 123.024 75.28984) (end 123.33984 74.974) (width 0.2) (layer "F.Cu") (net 5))
 (segment (start 122.1125 77.2) (end 122.501848 77.2) (width 0.2) (layer "F.Cu") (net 5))
 (segment (start 125.06016 79.626) (end 119.2635 79.626) (width 0.2) (layer "F.Cu") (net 5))
 (segment (start 125.06016 74.974) (end 125.376 75.28984) (width 0.2) (layer "F.Cu") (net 5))
 (segment (start 122.501848 77.2) (end 123.024 76.677848) (width 0.2) (layer "F.Cu") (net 5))
 (segment (start 123.024 76.677848) (end 123.024 75.28984) (width 0.2) (layer "F.Cu") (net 5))
 (segment (start 119.2635 79.626) (end 118.6 78.9625) (width 0.2) (layer "F.Cu") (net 5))
 (segment (start 125.376 79.31016) (end 125.06016 79.626) (width 0.2) (layer "F.Cu") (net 5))
 (segment (start 125.376 75.28984) (end 125.376 79.31016) (width 0.2) (layer "F.Cu") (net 5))
 (segment (start 121.474 77.474) (end 121.474 77.950848) (width 0.2) (layer "F.Cu") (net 8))
 (segment (start 121.474 77.950848) (end 122.285652 78.7625) (width 0.2) (layer "F.Cu") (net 8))
 (segment (start 120.6875 77.2) (end 121.2 77.2) (width 0.2) (layer "F.Cu") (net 8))
 (segment (start 121.2 77.2) (end 121.474 77.474) (width 0.2) (layer "F.Cu") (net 8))
 (segment (start 122.285652 78.7625) (end 124.2 78.7625) (width 0.2) (layer "F.Cu") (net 8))
 (segment (start 110.251 82.66284) (end 110.251 83.051) (width 0.2) (layer "F.Cu") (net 6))
 (segment (start 120.5865 75.174) (end 117.73984 75.174) (width 0.2) (layer "F.Cu") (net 6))
 (segment (start 108 82.6) (end 108 82) (width 0.2) (layer "F.Cu") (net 6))
 (segment (start 117.73984 75.174) (end 110.251 82.66284) (width 0.2) (layer "F.Cu") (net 6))
 (segment (start 108.451 83.051) (end 108 82.6) (width 0.2) (layer "F.Cu") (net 6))
 (segment (start 110.251 83.051) (end 108.451 83.051) (width 0.2) (layer "F.Cu") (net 6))
 (segment (start 122.1125 76.7) (end 120.5865 75.174) (width 0.2) (layer "F.Cu") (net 6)))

